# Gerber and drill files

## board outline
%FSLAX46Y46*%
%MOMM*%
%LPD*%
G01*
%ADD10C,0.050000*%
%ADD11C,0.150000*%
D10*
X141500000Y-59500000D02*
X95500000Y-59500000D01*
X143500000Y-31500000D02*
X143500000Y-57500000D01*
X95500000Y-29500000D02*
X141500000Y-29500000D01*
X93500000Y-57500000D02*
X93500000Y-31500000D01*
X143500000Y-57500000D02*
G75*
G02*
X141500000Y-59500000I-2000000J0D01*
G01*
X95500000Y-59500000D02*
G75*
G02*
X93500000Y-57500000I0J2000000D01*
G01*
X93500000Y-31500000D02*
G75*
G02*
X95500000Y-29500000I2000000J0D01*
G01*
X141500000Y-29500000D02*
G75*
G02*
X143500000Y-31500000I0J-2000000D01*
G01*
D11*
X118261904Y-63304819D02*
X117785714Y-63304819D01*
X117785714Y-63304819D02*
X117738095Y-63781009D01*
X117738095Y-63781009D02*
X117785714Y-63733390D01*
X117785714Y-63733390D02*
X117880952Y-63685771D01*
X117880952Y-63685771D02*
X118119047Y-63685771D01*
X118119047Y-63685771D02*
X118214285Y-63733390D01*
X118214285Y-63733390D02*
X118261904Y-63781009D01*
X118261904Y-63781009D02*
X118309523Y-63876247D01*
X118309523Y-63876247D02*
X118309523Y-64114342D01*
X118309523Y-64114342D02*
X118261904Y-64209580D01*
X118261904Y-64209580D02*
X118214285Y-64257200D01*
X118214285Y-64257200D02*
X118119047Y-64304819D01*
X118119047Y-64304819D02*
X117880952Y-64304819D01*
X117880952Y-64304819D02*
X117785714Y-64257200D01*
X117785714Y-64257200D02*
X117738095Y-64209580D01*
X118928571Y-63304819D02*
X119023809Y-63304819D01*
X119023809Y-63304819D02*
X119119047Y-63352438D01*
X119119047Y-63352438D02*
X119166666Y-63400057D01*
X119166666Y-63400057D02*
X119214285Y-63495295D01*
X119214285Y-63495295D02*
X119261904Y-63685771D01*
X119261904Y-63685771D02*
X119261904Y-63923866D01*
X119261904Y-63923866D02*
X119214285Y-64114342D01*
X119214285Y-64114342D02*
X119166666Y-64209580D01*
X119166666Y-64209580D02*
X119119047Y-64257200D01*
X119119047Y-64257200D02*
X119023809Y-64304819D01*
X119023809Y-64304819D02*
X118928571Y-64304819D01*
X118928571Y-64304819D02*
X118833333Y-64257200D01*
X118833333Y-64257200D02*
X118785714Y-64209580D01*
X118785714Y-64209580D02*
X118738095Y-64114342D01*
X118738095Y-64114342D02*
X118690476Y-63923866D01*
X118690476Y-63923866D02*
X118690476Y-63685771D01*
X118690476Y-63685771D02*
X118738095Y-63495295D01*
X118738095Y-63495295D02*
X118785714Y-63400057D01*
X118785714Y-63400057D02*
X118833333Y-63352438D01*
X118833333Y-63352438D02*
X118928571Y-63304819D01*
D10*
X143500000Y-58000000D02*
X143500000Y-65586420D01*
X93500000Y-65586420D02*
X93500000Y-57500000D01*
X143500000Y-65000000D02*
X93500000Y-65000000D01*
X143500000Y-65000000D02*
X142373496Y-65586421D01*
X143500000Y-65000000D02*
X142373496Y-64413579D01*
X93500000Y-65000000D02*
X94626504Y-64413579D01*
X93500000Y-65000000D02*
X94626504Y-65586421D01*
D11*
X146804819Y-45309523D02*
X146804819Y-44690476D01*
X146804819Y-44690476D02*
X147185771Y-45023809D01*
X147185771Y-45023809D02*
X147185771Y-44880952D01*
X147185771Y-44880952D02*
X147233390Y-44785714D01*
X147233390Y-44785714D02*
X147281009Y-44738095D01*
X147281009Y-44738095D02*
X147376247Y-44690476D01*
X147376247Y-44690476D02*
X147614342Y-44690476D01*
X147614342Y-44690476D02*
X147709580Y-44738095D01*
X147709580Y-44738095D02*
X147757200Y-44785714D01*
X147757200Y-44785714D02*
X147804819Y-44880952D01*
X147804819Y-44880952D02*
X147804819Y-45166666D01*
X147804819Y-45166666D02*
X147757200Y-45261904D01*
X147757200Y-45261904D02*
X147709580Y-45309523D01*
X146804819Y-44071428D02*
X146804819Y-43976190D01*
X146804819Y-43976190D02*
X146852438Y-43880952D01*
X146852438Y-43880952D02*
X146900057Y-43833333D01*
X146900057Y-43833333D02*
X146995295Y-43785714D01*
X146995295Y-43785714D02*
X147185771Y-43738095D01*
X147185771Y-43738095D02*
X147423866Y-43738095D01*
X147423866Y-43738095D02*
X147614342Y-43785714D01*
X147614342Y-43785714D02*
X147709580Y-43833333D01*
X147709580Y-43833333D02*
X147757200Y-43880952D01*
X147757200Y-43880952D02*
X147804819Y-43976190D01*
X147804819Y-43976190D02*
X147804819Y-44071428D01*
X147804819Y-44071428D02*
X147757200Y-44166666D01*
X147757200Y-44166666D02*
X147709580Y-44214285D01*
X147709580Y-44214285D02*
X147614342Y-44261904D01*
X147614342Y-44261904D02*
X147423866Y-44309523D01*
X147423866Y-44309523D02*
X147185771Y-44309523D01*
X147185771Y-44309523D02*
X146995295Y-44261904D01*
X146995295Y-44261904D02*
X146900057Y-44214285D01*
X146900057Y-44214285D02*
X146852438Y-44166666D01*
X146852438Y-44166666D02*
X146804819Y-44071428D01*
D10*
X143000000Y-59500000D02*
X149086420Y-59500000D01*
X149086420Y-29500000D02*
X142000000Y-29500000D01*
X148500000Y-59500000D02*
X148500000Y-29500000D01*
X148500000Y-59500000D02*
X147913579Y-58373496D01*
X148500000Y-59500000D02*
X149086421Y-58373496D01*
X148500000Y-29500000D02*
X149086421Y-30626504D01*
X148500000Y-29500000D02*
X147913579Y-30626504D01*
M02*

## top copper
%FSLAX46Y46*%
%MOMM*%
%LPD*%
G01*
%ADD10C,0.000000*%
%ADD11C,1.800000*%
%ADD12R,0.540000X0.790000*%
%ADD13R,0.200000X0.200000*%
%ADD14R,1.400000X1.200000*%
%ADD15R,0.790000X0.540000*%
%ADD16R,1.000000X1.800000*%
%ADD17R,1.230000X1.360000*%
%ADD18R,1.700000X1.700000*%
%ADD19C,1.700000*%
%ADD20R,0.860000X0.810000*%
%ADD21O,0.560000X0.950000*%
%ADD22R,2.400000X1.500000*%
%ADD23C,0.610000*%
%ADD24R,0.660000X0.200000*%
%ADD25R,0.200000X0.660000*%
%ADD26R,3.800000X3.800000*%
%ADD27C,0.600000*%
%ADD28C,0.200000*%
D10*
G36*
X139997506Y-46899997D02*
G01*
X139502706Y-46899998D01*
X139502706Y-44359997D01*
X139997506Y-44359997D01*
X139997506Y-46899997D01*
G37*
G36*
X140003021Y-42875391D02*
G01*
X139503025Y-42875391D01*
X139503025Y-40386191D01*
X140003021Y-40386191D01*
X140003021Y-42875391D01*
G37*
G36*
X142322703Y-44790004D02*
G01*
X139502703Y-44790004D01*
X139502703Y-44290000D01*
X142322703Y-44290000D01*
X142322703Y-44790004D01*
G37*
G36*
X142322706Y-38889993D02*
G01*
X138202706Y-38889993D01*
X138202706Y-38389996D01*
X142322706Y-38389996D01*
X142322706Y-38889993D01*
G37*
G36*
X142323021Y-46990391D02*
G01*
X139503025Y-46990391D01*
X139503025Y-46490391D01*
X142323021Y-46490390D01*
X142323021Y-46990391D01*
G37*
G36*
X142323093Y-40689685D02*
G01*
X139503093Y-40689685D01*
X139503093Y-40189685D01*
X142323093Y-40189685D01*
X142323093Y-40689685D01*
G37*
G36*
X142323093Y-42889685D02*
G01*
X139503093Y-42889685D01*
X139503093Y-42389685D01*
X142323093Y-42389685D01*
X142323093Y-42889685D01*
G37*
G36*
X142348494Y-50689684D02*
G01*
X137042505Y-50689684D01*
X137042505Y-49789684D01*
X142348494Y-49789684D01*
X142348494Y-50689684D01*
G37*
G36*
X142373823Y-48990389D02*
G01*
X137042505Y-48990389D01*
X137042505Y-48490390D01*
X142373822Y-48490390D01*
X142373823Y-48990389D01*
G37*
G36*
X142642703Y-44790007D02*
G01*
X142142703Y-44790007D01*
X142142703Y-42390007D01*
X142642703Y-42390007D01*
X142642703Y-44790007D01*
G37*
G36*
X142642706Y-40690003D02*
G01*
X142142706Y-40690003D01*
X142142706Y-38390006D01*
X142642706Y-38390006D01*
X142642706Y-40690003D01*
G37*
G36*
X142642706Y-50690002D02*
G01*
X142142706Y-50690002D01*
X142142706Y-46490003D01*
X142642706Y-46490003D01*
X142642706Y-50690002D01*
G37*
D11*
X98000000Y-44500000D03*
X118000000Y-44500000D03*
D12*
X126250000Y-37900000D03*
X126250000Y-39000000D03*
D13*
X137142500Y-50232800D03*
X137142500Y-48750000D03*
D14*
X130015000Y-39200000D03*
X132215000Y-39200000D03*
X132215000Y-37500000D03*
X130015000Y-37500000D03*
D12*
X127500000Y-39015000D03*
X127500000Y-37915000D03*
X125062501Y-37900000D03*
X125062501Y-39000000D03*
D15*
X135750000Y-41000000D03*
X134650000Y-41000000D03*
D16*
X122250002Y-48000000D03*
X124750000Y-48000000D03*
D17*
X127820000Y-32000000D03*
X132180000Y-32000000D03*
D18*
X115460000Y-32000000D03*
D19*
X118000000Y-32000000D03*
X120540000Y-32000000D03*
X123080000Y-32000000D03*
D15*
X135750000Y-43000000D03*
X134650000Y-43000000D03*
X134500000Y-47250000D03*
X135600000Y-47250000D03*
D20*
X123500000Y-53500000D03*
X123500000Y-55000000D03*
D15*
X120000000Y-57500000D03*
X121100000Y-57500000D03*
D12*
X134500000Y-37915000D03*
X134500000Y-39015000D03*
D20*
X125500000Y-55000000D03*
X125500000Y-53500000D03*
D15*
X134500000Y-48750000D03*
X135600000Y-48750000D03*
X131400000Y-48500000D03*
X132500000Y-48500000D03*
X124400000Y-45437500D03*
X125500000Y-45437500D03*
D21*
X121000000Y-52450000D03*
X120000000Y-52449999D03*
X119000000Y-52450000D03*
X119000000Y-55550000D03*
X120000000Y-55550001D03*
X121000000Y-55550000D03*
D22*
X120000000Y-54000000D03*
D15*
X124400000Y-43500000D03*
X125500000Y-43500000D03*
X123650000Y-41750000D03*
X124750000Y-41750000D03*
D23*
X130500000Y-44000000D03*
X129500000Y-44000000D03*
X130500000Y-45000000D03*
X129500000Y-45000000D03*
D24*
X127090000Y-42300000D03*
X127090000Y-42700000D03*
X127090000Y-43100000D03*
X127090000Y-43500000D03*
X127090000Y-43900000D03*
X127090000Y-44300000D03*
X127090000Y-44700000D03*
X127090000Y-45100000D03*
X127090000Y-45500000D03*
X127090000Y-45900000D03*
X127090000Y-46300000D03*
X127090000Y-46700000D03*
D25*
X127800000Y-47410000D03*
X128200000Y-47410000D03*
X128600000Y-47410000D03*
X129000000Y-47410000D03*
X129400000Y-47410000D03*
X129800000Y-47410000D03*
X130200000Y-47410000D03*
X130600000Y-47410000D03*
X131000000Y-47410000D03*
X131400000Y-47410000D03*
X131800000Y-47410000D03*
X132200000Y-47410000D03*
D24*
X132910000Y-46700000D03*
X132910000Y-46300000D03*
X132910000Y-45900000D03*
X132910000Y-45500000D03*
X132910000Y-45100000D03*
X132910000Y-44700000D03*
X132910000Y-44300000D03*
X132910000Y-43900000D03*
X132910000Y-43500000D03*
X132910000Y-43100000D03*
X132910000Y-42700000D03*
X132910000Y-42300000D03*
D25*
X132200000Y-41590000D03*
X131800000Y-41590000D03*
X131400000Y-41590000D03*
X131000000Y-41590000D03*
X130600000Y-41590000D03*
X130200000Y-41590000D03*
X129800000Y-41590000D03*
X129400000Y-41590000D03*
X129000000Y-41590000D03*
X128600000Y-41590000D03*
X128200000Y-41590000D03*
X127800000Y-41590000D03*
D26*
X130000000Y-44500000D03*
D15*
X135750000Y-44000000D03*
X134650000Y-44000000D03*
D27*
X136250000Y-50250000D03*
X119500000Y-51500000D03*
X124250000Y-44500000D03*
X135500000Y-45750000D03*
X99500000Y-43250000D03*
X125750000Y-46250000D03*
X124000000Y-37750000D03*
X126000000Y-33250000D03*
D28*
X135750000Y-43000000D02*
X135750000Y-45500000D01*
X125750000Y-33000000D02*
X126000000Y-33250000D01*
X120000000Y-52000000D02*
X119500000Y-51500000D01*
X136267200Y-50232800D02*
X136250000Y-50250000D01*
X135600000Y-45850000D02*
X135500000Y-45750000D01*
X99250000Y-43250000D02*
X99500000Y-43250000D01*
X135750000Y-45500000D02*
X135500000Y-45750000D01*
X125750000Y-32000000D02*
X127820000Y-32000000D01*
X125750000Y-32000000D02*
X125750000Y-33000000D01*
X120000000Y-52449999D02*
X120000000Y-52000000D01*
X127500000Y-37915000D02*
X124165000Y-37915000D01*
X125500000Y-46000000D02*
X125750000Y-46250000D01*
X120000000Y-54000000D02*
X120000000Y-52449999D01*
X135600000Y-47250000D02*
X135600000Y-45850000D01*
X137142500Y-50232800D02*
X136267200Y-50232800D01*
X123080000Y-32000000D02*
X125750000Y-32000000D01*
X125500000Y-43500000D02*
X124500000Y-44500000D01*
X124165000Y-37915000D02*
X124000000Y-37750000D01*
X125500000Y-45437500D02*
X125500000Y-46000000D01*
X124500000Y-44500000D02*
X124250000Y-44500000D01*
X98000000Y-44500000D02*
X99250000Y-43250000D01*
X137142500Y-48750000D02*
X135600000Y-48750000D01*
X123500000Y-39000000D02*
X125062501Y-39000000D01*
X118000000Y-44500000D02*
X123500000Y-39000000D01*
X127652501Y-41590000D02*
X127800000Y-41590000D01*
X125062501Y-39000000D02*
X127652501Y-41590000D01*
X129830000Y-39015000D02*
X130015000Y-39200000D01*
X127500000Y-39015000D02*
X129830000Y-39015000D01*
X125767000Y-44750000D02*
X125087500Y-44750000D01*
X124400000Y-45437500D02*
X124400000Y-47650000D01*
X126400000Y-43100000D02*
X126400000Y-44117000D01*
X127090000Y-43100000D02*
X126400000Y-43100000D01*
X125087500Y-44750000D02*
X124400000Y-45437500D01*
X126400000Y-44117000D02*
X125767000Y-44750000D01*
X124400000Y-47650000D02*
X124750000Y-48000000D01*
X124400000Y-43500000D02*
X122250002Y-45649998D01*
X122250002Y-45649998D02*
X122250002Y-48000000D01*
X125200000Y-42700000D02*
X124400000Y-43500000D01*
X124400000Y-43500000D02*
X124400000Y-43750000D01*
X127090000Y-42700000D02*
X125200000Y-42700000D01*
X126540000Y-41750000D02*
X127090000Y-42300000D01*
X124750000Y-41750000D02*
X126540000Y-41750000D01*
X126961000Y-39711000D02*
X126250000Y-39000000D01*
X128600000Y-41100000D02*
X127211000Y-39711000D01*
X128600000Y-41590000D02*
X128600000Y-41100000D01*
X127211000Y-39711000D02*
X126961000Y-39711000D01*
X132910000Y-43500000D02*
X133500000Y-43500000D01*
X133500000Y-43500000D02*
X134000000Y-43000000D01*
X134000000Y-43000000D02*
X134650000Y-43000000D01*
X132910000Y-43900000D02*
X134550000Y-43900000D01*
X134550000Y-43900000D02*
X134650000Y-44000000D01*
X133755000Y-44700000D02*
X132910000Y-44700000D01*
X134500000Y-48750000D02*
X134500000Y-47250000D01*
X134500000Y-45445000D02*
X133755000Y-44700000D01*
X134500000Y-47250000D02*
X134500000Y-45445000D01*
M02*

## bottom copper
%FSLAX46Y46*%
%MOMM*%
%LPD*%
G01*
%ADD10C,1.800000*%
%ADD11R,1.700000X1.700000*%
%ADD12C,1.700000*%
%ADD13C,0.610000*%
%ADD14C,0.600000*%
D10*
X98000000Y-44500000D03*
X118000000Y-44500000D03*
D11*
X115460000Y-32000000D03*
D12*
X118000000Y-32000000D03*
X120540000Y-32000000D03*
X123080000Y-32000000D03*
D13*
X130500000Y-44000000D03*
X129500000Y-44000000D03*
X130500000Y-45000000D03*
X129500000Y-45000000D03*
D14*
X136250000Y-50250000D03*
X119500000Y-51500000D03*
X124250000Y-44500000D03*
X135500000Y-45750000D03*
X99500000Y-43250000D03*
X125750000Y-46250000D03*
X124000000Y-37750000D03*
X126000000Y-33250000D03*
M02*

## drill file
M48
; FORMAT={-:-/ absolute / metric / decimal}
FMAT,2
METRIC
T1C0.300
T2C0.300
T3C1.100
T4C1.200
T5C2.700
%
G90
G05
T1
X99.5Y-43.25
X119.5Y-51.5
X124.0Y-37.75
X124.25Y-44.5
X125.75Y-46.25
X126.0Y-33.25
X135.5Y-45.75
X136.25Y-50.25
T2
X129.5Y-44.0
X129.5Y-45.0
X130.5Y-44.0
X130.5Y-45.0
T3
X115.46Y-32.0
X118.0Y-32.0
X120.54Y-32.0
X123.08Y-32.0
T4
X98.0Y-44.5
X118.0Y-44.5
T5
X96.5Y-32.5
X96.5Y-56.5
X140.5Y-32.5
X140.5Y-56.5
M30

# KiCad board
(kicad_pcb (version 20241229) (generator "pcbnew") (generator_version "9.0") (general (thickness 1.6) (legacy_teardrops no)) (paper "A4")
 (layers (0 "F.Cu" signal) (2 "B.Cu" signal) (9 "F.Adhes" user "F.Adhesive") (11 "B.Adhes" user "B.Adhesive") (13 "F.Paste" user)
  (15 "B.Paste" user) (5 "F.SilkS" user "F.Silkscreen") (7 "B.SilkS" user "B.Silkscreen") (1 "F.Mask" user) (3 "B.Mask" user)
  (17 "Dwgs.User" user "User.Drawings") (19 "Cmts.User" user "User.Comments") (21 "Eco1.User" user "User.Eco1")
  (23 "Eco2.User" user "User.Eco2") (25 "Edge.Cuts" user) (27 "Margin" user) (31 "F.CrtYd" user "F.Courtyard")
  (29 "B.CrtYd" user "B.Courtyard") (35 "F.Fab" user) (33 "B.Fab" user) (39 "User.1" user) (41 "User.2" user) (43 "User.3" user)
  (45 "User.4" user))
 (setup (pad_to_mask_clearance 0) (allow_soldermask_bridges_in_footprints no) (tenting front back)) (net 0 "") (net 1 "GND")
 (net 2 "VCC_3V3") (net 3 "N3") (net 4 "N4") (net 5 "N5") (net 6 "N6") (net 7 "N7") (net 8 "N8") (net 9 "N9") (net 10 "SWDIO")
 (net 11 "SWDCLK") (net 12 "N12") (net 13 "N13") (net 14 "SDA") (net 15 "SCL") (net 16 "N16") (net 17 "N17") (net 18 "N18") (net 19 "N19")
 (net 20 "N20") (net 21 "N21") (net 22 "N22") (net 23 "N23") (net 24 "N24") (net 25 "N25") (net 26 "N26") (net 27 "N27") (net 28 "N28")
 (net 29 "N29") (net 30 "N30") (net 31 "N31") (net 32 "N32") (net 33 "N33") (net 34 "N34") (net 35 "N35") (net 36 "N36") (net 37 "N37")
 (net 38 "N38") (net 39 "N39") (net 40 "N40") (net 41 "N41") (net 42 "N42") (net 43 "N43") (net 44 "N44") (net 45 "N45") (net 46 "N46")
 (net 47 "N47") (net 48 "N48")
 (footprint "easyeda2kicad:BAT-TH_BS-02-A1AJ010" (layer "F.Cu") (at 108 44.5)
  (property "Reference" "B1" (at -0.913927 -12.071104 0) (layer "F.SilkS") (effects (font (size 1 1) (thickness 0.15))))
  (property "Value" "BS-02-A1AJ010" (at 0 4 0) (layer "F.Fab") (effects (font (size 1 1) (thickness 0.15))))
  (pad "1" thru_hole circle (at -10 0) (size 1.8 1.8) (drill 1.199998) (layers "*.Cu" "*.Mask") (remove_unused_layers no) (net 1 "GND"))
  (pad "2" thru_hole circle (at 10 0) (size 1.8 1.8) (drill 1.199998) (layers "*.Cu" "*.Mask") (remove_unused_layers no) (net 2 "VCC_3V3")))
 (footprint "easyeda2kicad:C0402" (layer "F.Cu") (at 126.25 38.45 -90)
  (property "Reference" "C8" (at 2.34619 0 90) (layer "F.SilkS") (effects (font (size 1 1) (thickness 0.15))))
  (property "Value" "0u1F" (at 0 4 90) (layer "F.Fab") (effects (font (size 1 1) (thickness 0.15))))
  (pad "1" smd rect (at -0.55 0 270) (size 0.79 0.54) (layers "F.Cu" "F.Mask" "F.Paste") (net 1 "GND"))
  (pad "2" smd rect (at 0.55 0 270) (size 0.79 0.54) (layers "F.Cu" "F.Mask" "F.Paste") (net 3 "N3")))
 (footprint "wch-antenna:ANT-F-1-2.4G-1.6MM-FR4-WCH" (layer "F.Cu") (at 140 44.6225 -90)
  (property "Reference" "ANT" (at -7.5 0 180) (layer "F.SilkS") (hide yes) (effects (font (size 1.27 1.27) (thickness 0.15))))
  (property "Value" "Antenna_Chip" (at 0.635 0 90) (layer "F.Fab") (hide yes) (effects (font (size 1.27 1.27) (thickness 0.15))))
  (fp_poly
   (pts (xy 2.277497 0.002494) (xy -0.262503 0.002494) (xy -0.262503 0.497294) (xy 2.277498 0.497294)) (stroke (width 0) (type solid))
   (fill yes) (layer "F.Cu"))
  (fp_poly
   (pts (xy -1.747109 -0.003021) (xy -4.236309 -0.003021) (xy -4.236309 0.496975) (xy -1.747109 0.496975)) (stroke (width 0) (type solid))
   (fill yes) (layer "F.Cu"))
  (fp_poly
   (pts (xy 0.167504 -2.322703) (xy -0.3325 -2.322703) (xy -0.3325 0.497297) (xy 0.167504 0.497297)) (stroke (width 0) (type solid))
   (fill yes) (layer "F.Cu"))
  (fp_poly
   (pts (xy -5.732507 -2.322706) (xy -6.232504 -2.322706) (xy -6.232504 1.797294) (xy -5.732507 1.797294)) (stroke (width 0) (type solid))
   (fill yes) (layer "F.Cu"))
  (fp_poly
   (pts (xy 2.367891 -2.323021) (xy 1.86789 -2.323021) (xy 1.867891 0.496975) (xy 2.367891 0.496975)) (stroke (width 0) (type solid))
   (fill yes) (layer "F.Cu"))
  (fp_poly
   (pts (xy -3.932815 -2.323093) (xy -4.432815 -2.323093) (xy -4.432815 0.496907) (xy -3.932815 0.496907)) (stroke (width 0) (type solid))
   (fill yes) (layer "F.Cu"))
  (fp_poly
   (pts (xy -1.732815 -2.323093) (xy -2.232815 -2.323093) (xy -2.232815 0.496907) (xy -1.732815 0.496907)) (stroke (width 0) (type solid))
   (fill yes) (layer "F.Cu"))
  (fp_poly
   (pts (xy 6.067184 -2.348494) (xy 5.167184 -2.348494) (xy 5.167184 2.957495) (xy 6.067184 2.957495)) (stroke (width 0) (type solid))
   (fill yes) (layer "F.Cu"))
  (fp_poly
   (pts (xy 4.367889 -2.373823) (xy 3.86789 -2.373822) (xy 3.86789 2.957495) (xy 4.367889 2.957495)) (stroke (width 0) (type solid))
   (fill yes) (layer "F.Cu"))
  (fp_poly
   (pts (xy 0.167507 -2.642703) (xy -2.232493 -2.642703) (xy -2.232493 -2.142703) (xy 0.167507 -2.142703)) (stroke (width 0) (type solid))
   (fill yes) (layer "F.Cu"))
  (fp_poly
   (pts (xy -3.932497 -2.642706) (xy -6.232494 -2.642706) (xy -6.232494 -2.142706) (xy -3.932497 -2.142706)) (stroke (width 0) (type solid))
   (fill yes) (layer "F.Cu"))
  (fp_poly
   (pts (xy 6.067502 -2.642706) (xy 1.867503 -2.642706) (xy 1.867503 -2.142706) (xy 6.067502 -2.142706)) (stroke (width 0) (type solid))
   (fill yes) (layer "F.Cu"))
  (pad "1" smd rect (at 5.6103 2.8575) (size 0.2 0.2) (layers "F.Cu") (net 1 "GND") (solder_mask_margin 0.1016))
  (pad "2" smd rect (at 4.1275 2.8575) (size 0.2 0.2) (layers "F.Cu") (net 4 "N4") (solder_mask_margin 0.1016)))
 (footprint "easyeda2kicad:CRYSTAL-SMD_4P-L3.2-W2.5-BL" (layer "F.Cu") (at 131.115 38.35)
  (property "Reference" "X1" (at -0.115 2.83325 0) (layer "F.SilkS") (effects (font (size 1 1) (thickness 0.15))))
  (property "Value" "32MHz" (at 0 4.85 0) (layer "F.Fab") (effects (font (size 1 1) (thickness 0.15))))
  (pad "1" smd rect (at -1.1 0.85) (size 1.4 1.2) (layers "F.Cu" "F.Mask" "F.Paste") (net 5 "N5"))
  (pad "2" smd rect (at 1.1 0.85) (size 1.4 1.2) (layers "F.Cu" "F.Mask" "F.Paste") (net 1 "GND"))
  (pad "3" smd rect (at 1.1 -0.85) (size 1.4 1.2) (layers "F.Cu" "F.Mask" "F.Paste") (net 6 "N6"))
  (pad "4" smd rect (at -1.1 -0.85) (size 1.4 1.2) (layers "F.Cu" "F.Mask" "F.Paste") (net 1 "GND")))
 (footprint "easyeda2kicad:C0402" (layer "F.Cu") (at 127.5 38.465 90)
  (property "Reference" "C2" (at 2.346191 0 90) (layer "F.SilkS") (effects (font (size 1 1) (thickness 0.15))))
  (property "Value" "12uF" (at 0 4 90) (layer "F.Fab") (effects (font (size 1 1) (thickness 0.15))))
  (pad "1" smd rect (at -0.55 0 90) (size 0.79 0.54) (layers "F.Cu" "F.Mask" "F.Paste") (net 5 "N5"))
  (pad "2" smd rect (at 0.55 0 90) (size 0.79 0.54) (layers "F.Cu" "F.Mask" "F.Paste") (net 1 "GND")))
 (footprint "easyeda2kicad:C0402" (layer "F.Cu") (at 125.062501 38.45 -90)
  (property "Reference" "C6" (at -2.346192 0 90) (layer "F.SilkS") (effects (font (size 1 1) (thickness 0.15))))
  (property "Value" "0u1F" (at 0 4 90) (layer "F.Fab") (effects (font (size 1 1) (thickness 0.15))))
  (pad "1" smd rect (at -0.55 0 270) (size 0.79 0.54) (layers "F.Cu" "F.Mask" "F.Paste") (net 1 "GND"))
  (pad "2" smd rect (at 0.55 0 270) (size 0.79 0.54) (layers "F.Cu" "F.Mask" "F.Paste") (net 2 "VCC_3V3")))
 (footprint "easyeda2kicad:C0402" (layer "F.Cu") (at 135.2 41 180)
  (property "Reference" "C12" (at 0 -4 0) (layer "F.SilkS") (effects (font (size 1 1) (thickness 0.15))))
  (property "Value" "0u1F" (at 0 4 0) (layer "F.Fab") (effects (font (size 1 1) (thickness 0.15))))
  (pad "1" smd rect (at -0.55 0 180) (size 0.79 0.54) (layers "F.Cu" "F.Mask" "F.Paste") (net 1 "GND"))
  (pad "2" smd rect (at 0.55 0 180) (size 0.79 0.54) (layers "F.Cu" "F.Mask" "F.Paste") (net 2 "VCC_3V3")))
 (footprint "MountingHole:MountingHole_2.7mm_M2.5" (layer "F.Cu") (at 140.5 32.5)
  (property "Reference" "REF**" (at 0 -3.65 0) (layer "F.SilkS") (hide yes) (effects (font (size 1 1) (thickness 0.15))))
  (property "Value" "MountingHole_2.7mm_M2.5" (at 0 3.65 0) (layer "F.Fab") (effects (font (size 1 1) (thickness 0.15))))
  (pad "" np_thru_hole circle (at 0 0) (size 2.7 2.7) (drill 2.7) (layers "*.Cu" "*.Mask")))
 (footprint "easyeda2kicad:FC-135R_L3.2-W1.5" (layer "F.Cu") (at 123.500001 48)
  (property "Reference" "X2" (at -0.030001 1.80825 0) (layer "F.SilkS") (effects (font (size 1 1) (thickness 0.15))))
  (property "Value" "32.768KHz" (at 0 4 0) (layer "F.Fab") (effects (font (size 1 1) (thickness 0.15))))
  (pad "1" smd rect (at -1.249999 0 90) (size 1.8 1) (layers "F.Cu" "F.Mask" "F.Paste") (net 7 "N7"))
  (pad "2" smd rect (at 1.249999 0 90) (size 1.8 1) (layers "F.Cu" "F.Mask" "F.Paste") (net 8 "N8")))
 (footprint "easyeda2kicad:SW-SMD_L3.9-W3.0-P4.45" (layer "F.Cu") (at 130 32)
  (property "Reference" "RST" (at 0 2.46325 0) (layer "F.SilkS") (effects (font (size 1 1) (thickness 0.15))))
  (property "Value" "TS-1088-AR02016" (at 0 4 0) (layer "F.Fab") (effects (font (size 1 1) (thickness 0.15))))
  (pad "1" smd rect (at -2.18 0) (size 1.23 1.36) (layers "F.Cu" "F.Mask" "F.Paste") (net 1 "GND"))
  (pad "2" smd rect (at 2.18 0) (size 1.23 1.36) (layers "F.Cu" "F.Mask" "F.Paste") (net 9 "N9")))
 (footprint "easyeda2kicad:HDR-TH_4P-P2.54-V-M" (layer "F.Cu") (at 119.27 32)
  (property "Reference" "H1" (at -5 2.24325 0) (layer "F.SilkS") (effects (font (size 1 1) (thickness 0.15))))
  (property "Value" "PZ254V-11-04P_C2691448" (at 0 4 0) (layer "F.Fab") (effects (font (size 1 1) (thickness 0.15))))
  (pad "1" thru_hole rect (at -3.81 0) (size 1.7 1.7) (drill 1.100023) (layers "*.Cu" "*.Mask") (remove_unused_layers no) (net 2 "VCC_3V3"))
  (pad "2" thru_hole circle (at -1.27 0) (size 1.7 1.7) (drill 1.100023) (layers "*.Cu" "*.Mask") (remove_unused_layers no) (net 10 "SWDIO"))
  (pad "3" thru_hole circle (at 1.27 0) (size 1.7 1.7) (drill 1.100023) (layers "*.Cu" "*.Mask") (remove_unused_layers no) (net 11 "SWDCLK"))
  (pad "4" thru_hole circle (at 3.81 0) (size 1.7 1.7) (drill 1.100023) (layers "*.Cu" "*.Mask") (remove_unused_layers no) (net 1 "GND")))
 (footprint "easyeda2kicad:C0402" (layer "F.Cu") (at 135.2 43 180)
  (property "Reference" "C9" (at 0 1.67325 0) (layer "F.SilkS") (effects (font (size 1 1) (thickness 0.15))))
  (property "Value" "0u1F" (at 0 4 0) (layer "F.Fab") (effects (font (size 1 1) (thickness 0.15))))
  (pad "1" smd rect (at -0.55 0 180) (size 0.79 0.54) (layers "F.Cu" "F.Mask" "F.Paste") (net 1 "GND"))
  (pad "2" smd rect (at 0.55 0 180) (size 0.79 0.54) (layers "F.Cu" "F.Mask" "F.Paste") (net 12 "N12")))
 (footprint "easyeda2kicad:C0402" (layer "F.Cu") (at 135.05 47.25)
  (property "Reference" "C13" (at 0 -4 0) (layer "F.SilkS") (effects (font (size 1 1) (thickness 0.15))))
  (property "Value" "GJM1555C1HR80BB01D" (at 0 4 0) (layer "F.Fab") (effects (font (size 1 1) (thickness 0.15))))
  (pad "1" smd rect (at -0.55 0) (size 0.79 0.54) (layers "F.Cu" "F.Mask" "F.Paste") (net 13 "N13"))
  (pad "2" smd rect (at 0.55 0) (size 0.79 0.54) (layers "F.Cu" "F.Mask" "F.Paste") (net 1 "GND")))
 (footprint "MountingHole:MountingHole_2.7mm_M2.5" (layer "F.Cu") (at 140.5 56.5)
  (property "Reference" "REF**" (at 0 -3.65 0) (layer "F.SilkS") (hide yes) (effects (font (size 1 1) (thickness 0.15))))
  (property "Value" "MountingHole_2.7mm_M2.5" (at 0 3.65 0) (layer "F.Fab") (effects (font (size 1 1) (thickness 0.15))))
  (pad "" np_thru_hole circle (at 0 0) (size 2.7 2.7) (drill 2.7) (layers "*.Cu" "*.Mask")))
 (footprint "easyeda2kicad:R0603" (layer "F.Cu") (at 123.5 54.25 -90)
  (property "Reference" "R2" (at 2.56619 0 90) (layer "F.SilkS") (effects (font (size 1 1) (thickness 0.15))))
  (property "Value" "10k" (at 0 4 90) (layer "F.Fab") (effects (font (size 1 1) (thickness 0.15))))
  (pad "1" smd rect (at -0.75 0 270) (size 0.81 0.86) (layers "F.Cu" "F.Mask" "F.Paste") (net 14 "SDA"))
  (pad "2" smd rect (at 0.75 0 270) (size 0.81 0.86) (layers "F.Cu" "F.Mask" "F.Paste") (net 2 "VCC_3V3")))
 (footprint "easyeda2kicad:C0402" (layer "F.Cu") (at 120.55 57.5)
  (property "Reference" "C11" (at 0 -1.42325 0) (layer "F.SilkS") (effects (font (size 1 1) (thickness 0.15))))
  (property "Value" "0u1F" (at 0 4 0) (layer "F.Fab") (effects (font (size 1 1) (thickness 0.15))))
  (pad "1" smd rect (at -0.55 0) (size 0.79 0.54) (layers "F.Cu" "F.Mask" "F.Paste") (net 1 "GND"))
  (pad "2" smd rect (at 0.55 0) (size 0.79 0.54) (layers "F.Cu" "F.Mask" "F.Paste") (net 2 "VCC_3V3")))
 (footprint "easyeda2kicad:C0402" (layer "F.Cu") (at 134.5 38.465 -90)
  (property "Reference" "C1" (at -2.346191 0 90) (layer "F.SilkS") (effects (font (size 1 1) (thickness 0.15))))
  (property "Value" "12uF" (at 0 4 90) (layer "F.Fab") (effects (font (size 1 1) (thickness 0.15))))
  (pad "1" smd rect (at -0.55 0 270) (size 0.79 0.54) (layers "F.Cu" "F.Mask" "F.Paste") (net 6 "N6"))
  (pad "2" smd rect (at 0.55 0 270) (size 0.79 0.54) (layers "F.Cu" "F.Mask" "F.Paste") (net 1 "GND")))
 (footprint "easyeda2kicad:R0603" (layer "F.Cu") (at 125.5 54.25 90)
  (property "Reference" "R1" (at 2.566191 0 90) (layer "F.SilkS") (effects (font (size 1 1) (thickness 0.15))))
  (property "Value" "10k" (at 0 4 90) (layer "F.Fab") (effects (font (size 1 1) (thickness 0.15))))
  (pad "1" smd rect (at -0.75 0 90) (size 0.81 0.86) (layers "F.Cu" "F.Mask" "F.Paste") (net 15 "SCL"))
  (pad "2" smd rect (at 0.75 0 90) (size 0.81 0.86) (layers "F.Cu" "F.Mask" "F.Paste") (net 2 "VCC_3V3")))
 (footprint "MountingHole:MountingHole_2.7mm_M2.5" (layer "F.Cu") (at 96.5 32.5)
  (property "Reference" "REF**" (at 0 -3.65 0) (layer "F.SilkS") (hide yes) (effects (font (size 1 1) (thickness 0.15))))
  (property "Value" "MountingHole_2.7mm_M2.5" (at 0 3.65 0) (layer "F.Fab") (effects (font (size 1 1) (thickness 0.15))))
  (pad "" np_thru_hole circle (at 0 0) (size 2.7 2.7) (drill 2.7) (layers "*.Cu" "*.Mask")))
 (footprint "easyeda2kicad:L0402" (layer "F.Cu") (at 135.05 48.75)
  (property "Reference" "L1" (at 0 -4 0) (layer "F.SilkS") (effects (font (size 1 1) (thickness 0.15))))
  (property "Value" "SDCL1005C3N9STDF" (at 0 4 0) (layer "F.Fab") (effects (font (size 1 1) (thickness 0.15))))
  (pad "1" smd rect (at -0.55 0) (size 0.79 0.54) (layers "F.Cu" "F.Mask" "F.Paste") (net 13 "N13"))
  (pad "2" smd rect (at 0.55 0) (size 0.79 0.54) (layers "F.Cu" "F.Mask" "F.Paste") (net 4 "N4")))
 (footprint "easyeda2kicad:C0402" (layer "F.Cu") (at 131.95 48.5)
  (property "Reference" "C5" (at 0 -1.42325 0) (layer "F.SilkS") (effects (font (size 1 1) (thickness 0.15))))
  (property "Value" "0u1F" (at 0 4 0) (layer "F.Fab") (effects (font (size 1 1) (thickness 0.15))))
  (pad "1" smd rect (at -0.55 0) (size 0.79 0.54) (layers "F.Cu" "F.Mask" "F.Paste") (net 1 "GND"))
  (pad "2" smd rect (at 0.55 0) (size 0.79 0.54) (layers "F.Cu" "F.Mask" "F.Paste") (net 2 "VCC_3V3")))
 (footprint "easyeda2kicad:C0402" (layer "F.Cu") (at 124.95 45.4375)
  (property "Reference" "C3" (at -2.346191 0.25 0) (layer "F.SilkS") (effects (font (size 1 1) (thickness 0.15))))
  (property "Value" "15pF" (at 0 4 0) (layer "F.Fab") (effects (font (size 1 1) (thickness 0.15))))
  (pad "1" smd rect (at -0.55 0) (size 0.79 0.54) (layers "F.Cu" "F.Mask" "F.Paste") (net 8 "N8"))
  (pad "2" smd rect (at 0.55 0) (size 0.79 0.54) (layers "F.Cu" "F.Mask" "F.Paste") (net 1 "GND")))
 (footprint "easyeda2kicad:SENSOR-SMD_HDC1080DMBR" (layer "F.Cu") (at 120 54 -90)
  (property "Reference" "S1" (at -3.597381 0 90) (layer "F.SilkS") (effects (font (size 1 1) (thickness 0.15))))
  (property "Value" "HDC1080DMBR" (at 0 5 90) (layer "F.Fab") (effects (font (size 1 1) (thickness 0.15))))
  (pad "1" smd oval (at -1.55 -1 270) (size 0.95 0.56) (layers "F.Cu" "F.Mask" "F.Paste") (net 14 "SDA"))
  (pad "2" smd oval (at -1.550001 0 270) (size 0.95 0.56) (layers "F.Cu" "F.Mask" "F.Paste") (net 1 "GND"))
  (pad "3" smd oval (at -1.55 1 270) (size 0.95 0.56) (layers "F.Cu" "F.Mask" "F.Paste") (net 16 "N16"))
  (pad "4" smd oval (at 1.55 1 270) (size 0.95 0.56) (layers "F.Cu" "F.Mask" "F.Paste") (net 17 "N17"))
  (pad "5" smd oval (at 1.550001 0 270) (size 0.95 0.56) (layers "F.Cu" "F.Mask" "F.Paste") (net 2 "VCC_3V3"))
  (pad "6" smd oval (at 1.55 -1 270) (size 0.95 0.56) (layers "F.Cu" "F.Mask" "F.Paste") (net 15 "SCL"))
  (pad "7" smd rect (at 0 0 270) (size 1.5 2.4) (layers "F.Cu" "F.Mask" "F.Paste") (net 1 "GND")))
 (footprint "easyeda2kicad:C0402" (layer "F.Cu") (at 124.95 43.5)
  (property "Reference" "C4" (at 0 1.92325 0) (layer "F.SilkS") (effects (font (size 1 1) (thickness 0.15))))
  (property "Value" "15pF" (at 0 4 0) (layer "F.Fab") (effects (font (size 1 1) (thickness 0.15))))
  (pad "1" smd rect (at -0.55 0) (size 0.79 0.54) (layers "F.Cu" "F.Mask" "F.Paste") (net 7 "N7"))
  (pad "2" smd rect (at 0.55 0) (size 0.79 0.54) (layers "F.Cu" "F.Mask" "F.Paste") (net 1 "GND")))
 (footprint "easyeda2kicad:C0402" (layer "F.Cu") (at 124.2 41.75)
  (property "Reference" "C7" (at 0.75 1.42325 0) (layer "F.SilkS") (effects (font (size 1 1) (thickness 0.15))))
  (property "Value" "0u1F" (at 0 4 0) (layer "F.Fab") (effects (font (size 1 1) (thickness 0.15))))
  (pad "1" smd rect (at -0.55 0) (size 0.79 0.54) (layers "F.Cu" "F.Mask" "F.Paste") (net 1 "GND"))
  (pad "2" smd rect (at 0.55 0) (size 0.79 0.54) (layers "F.Cu" "F.Mask" "F.Paste") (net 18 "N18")))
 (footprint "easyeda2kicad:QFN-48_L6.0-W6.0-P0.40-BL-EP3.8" (layer "F.Cu") (at 130 44.5 -90)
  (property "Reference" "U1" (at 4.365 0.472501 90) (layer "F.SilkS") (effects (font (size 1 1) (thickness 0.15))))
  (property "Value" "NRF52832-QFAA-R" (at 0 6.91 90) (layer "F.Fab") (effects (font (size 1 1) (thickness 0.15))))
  (pad "" thru_hole circle (at -0.5 -0.5 270) (size 0.61 0.61) (drill 0.3) (layers "*.Cu" "*.Paste" "*.Mask") (remove_unused_layers no))
  (pad "" thru_hole circle (at -0.5 0.5 270) (size 0.61 0.61) (drill 0.3) (layers "*.Cu" "*.Paste" "*.Mask") (remove_unused_layers no))
  (pad "" thru_hole circle (at 0.5 -0.5 270) (size 0.61 0.61) (drill 0.3) (layers "*.Cu" "*.Paste" "*.Mask") (remove_unused_layers no))
  (pad "" thru_hole circle (at 0.5 0.5 270) (size 0.61 0.61) (drill 0.3) (layers "*.Cu" "*.Paste" "*.Mask") (remove_unused_layers no))
  (pad "1" smd rect (at -2.2 2.91 270) (size 0.2 0.66) (layers "F.Cu" "F.Mask" "F.Paste") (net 18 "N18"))
  (pad "2" smd rect (at -1.8 2.91 270) (size 0.2 0.66) (layers "F.Cu" "F.Mask" "F.Paste") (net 7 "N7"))
  (pad "3" smd rect (at -1.4 2.91 270) (size 0.2 0.66) (layers "F.Cu" "F.Mask" "F.Paste") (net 8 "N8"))
  (pad "4" smd rect (at -1 2.91 270) (size 0.2 0.66) (layers "F.Cu" "F.Mask" "F.Paste") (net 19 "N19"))
  (pad "5" smd rect (at -0.6 2.91 270) (size 0.2 0.66) (layers "F.Cu" "F.Mask" "F.Paste") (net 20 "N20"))
  (pad "6" smd rect (at -0.2 2.91 270) (size 0.2 0.66) (layers "F.Cu" "F.Mask" "F.Paste") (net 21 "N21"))
  (pad "7" smd rect (at 0.2 2.91 270) (size 0.2 0.66) (layers "F.Cu" "F.Mask" "F.Paste") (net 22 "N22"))
  (pad "8" smd rect (at 0.6 2.91 270) (size 0.2 0.66) (layers "F.Cu" "F.Mask" "F.Paste") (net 14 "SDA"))
  (pad "9" smd rect (at 1 2.91 270) (size 0.2 0.66) (layers "F.Cu" "F.Mask" "F.Paste") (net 15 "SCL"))
  (pad "10" smd rect (at 1.4 2.91 270) (size 0.2 0.66) (layers "F.Cu" "F.Mask" "F.Paste") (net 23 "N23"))
  (pad "11" smd rect (at 1.8 2.91 270) (size 0.2 0.66) (layers "F.Cu" "F.Mask" "F.Paste") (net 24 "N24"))
  (pad "12" smd rect (at 2.2 2.91 270) (size 0.2 0.66) (layers "F.Cu" "F.Mask" "F.Paste") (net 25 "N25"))
  (pad "13" smd rect (at 2.91 2.2 270) (size 0.66 0.2) (layers "F.Cu" "F.Mask" "F.Paste") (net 2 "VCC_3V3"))
  (pad "14" smd rect (at 2.91 1.8 270) (size 0.66 0.2) (layers "F.Cu" "F.Mask" "F.Paste") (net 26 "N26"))
  (pad "15" smd rect (at 2.91 1.4 270) (size 0.66 0.2) (layers "F.Cu" "F.Mask" "F.Paste") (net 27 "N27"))
  (pad "16" smd rect (at 2.91 1 270) (size 0.66 0.2) (layers "F.Cu" "F.Mask" "F.Paste") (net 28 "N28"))
  (pad "17" smd rect (at 2.91 0.6 270) (size 0.66 0.2) (layers "F.Cu" "F.Mask" "F.Paste") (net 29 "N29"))
  (pad "18" smd rect (at 2.91 0.2 270) (size 0.66 0.2) (layers "F.Cu" "F.Mask" "F.Paste") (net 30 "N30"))
  (pad "19" smd rect (at 2.91 -0.2 270) (size 0.66 0.2) (layers "F.Cu" "F.Mask" "F.Paste") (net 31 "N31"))
  (pad "20" smd rect (at 2.91 -0.6 270) (size 0.66 0.2) (layers "F.Cu" "F.Mask" "F.Paste") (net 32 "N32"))
  (pad "21" smd rect (at 2.91 -1 270) (size 0.66 0.2) (layers "F.Cu" "F.Mask" "F.Paste") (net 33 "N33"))
  (pad "22" smd rect (at 2.91 -1.4 270) (size 0.66 0.2) (layers "F.Cu" "F.Mask" "F.Paste") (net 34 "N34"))
  (pad "23" smd rect (at 2.91 -1.8 270) (size 0.66 0.2) (layers "F.Cu" "F.Mask" "F.Paste") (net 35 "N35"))
  (pad "24" smd rect (at 2.91 -2.2 270) (size 0.66 0.2) (layers "F.Cu" "F.Mask" "F.Paste") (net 9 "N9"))
  (pad "25" smd rect (at 2.2 -2.91 270) (size 0.2 0.66) (layers "F.Cu" "F.Mask" "F.Paste") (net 11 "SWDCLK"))
  (pad "26" smd rect (at 1.8 -2.91 270) (size 0.2 0.66) (layers "F.Cu" "F.Mask" "F.Paste") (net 10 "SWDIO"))
  (pad "27" smd rect (at 1.4 -2.91 270) (size 0.2 0.66) (layers "F.Cu" "F.Mask" "F.Paste") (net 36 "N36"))
  (pad "28" smd rect (at 1 -2.91 270) (size 0.2 0.66) (layers "F.Cu" "F.Mask" "F.Paste") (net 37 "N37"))
  (pad "29" smd rect (at 0.6 -2.91 270) (size 0.2 0.66) (layers "F.Cu" "F.Mask" "F.Paste") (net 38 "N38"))
  (pad "30" smd rect (at 0.2 -2.91 270) (size 0.2 0.66) (layers "F.Cu" "F.Mask" "F.Paste") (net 13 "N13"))
  (pad "31" smd rect (at -0.2 -2.91 270) (size 0.2 0.66) (layers "F.Cu" "F.Mask" "F.Paste") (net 1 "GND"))
  (pad "32" smd rect (at -0.6 -2.91 270) (size 0.2 0.66) (layers "F.Cu" "F.Mask" "F.Paste") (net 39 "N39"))
  (pad "33" smd rect (at -1 -2.91 270) (size 0.2 0.66) (layers "F.Cu" "F.Mask" "F.Paste") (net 12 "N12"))
  (pad "34" smd rect (at -1.4 -2.91 270) (size 0.2 0.66) (layers "F.Cu" "F.Mask" "F.Paste") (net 5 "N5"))
  (pad "35" smd rect (at -1.8 -2.91 270) (size 0.2 0.66) (layers "F.Cu" "F.Mask" "F.Paste") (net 6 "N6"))
  (pad "36" smd rect (at -2.2 -2.91 270) (size 0.2 0.66) (layers "F.Cu" "F.Mask" "F.Paste") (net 2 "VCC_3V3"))
  (pad "37" smd rect (at -2.91 -2.2 270) (size 0.66 0.2) (layers "F.Cu" "F.Mask" "F.Paste") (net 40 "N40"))
  (pad "38" smd rect (at -2.91 -1.8 270) (size 0.66 0.2) (layers "F.Cu" "F.Mask" "F.Paste") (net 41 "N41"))
  (pad "39" smd rect (at -2.91 -1.4 270) (size 0.66 0.2) (layers "F.Cu" "F.Mask" "F.Paste") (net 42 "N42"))
  (pad "40" smd rect (at -2.91 -1 270) (size 0.66 0.2) (layers "F.Cu" "F.Mask" "F.Paste") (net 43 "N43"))
  (pad "41" smd rect (at -2.91 -0.6 270) (size 0.66 0.2) (layers "F.Cu" "F.Mask" "F.Paste") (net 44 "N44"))
  (pad "42" smd rect (at -2.91 -0.2 270) (size 0.66 0.2) (layers "F.Cu" "F.Mask" "F.Paste") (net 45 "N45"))
  (pad "43" smd rect (at -2.91 0.2 270) (size 0.66 0.2) (layers "F.Cu" "F.Mask" "F.Paste") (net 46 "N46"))
  (pad "44" smd rect (at -2.91 0.6 270) (size 0.66 0.2) (layers "F.Cu" "F.Mask" "F.Paste") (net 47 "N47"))
  (pad "45" smd rect (at -2.91 1 270) (size 0.66 0.2) (layers "F.Cu" "F.Mask" "F.Paste") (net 1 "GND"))
  (pad "46" smd rect (at -2.91 1.4 270) (size 0.66 0.2) (layers "F.Cu" "F.Mask" "F.Paste") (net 3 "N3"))
  (pad "47" smd rect (at -2.91 1.8 270) (size 0.66 0.2) (layers "F.Cu" "F.Mask" "F.Paste") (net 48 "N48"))
  (pad "48" smd rect (at -2.91 2.2 270) (size 0.66 0.2) (layers "F.Cu" "F.Mask" "F.Paste") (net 2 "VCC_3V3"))
  (pad "49" smd rect (at 0 0 270) (size 3.8 3.8) (layers "F.Cu" "F.Mask" "F.Paste") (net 1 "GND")))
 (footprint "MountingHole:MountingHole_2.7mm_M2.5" (layer "F.Cu") (at 96.5 56.5)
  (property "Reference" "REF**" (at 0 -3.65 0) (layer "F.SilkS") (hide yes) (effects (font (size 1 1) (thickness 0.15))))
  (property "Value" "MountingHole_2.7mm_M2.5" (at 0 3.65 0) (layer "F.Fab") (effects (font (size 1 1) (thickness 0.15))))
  (pad "" np_thru_hole circle (at 0 0) (size 2.7 2.7) (drill 2.7) (layers "*.Cu" "*.Mask")))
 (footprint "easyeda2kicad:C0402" (layer "F.Cu") (at 135.2 44 180)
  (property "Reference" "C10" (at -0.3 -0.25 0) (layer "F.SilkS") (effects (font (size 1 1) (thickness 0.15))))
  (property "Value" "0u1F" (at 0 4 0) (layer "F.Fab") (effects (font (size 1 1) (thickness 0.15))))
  (pad "1" smd rect (at -0.55 0 180) (size 0.79 0.54) (layers "F.Cu" "F.Mask" "F.Paste") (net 1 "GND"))
  (pad "2" smd rect (at 0.55 0 180) (size 0.79 0.54) (layers "F.Cu" "F.Mask" "F.Paste") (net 39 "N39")))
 (gr_line (start 141.5 59.5) (end 95.5 59.5) (stroke (width 0.05) (type default)) (layer "Edge.Cuts"))
 (gr_line (start 143.5 31.5) (end 143.5 57.5) (stroke (width 0.05) (type default)) (layer "Edge.Cuts"))
 (gr_line (start 95.5 29.5) (end 141.5 29.5) (stroke (width 0.05) (type default)) (layer "Edge.Cuts"))
 (gr_line (start 93.5 57.5) (end 93.5 31.5) (stroke (width 0.05) (type default)) (layer "Edge.Cuts"))
 (gr_arc (start 143.5 57.5) (mid 142.914214 58.914214) (end 141.5 59.5) (stroke (width 0.05) (type default)) (layer "Edge.Cuts"))
 (gr_arc (start 95.5 59.5) (mid 94.085786 58.914214) (end 93.5 57.5) (stroke (width 0.05) (type default)) (layer "Edge.Cuts"))
 (gr_arc (start 93.5 31.5) (mid 94.085786 30.085786) (end 95.5 29.5) (stroke (width 0.05) (type default)) (layer "Edge.Cuts"))
 (gr_arc (start 141.5 29.5) (mid 142.914214 30.085786) (end 143.5 31.5) (stroke (width 0.05) (type default)) (layer "Edge.Cuts"))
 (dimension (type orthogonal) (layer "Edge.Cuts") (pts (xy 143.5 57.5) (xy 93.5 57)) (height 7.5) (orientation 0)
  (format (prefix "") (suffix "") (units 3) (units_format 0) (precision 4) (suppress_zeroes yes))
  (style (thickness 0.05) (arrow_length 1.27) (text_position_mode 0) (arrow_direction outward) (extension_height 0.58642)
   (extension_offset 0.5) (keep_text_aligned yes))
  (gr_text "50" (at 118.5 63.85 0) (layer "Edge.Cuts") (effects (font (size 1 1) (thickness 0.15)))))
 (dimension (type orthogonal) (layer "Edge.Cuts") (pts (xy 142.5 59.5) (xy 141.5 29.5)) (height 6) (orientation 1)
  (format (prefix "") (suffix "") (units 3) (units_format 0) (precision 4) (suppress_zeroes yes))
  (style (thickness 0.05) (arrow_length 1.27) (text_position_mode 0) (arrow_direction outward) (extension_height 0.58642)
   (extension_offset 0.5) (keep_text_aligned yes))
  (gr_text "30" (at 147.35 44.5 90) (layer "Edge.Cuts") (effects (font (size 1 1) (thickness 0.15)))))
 (segment (start 135.75 43) (end 135.75 45.5) (width 0.2) (layer "F.Cu") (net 1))
 (segment (start 125.75 33) (end 126 33.25) (width 0.2) (layer "F.Cu") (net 1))
 (segment (start 120 52) (end 119.5 51.5) (width 0.2) (layer "F.Cu") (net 1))
 (segment (start 136.2672 50.2328) (end 136.25 50.25) (width 0.2) (layer "F.Cu") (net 1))
 (segment (start 135.6 45.85) (end 135.5 45.75) (width 0.2) (layer "F.Cu") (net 1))
 (segment (start 99.25 43.25) (end 99.5 43.25) (width 0.2) (layer "F.Cu") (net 1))
 (segment (start 135.75 45.5) (end 135.5 45.75) (width 0.2) (layer "F.Cu") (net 1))
 (segment (start 125.75 32) (end 127.82 32) (width 0.2) (layer "F.Cu") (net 1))
 (segment (start 125.75 32) (end 125.75 33) (width 0.2) (layer "F.Cu") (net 1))
 (segment (start 120 52.449999) (end 120 52) (width 0.2) (layer "F.Cu") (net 1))
 (segment (start 127.5 37.915) (end 124.165 37.915) (width 0.2) (layer "F.Cu") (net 1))
 (segment (start 125.5 46) (end 125.75 46.25) (width 0.2) (layer "F.Cu") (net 1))
 (segment (start 120 54) (end 120 52.449999) (width 0.2) (layer "F.Cu") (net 1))
 (segment (start 135.6 47.25) (end 135.6 45.85) (width 0.2) (layer "F.Cu") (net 1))
 (segment (start 137.1425 50.2328) (end 136.2672 50.2328) (width 0.2) (layer "F.Cu") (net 1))
 (segment (start 123.08 32) (end 125.75 32) (width 0.2) (layer "F.Cu") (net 1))
 (segment (start 125.5 43.5) (end 124.5 44.5) (width 0.2) (layer "F.Cu") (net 1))
 (segment (start 124.165 37.915) (end 124 37.75) (width 0.2) (layer "F.Cu") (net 1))
 (segment (start 125.5 45.4375) (end 125.5 46) (width 0.2) (layer "F.Cu") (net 1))
 (segment (start 124.5 44.5) (end 124.25 44.5) (width 0.2) (layer "F.Cu") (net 1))
 (segment (start 98 44.5) (end 99.25 43.25) (width 0.2) (layer "F.Cu") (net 1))
 (via (at 136.25 50.25) (size 0.6) (drill 0.3) (layers "F.Cu" "B.Cu") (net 1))
 (via (at 119.5 51.5) (size 0.6) (drill 0.3) (layers "F.Cu" "B.Cu") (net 1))
 (via (at 124.25 44.5) (size 0.6) (drill 0.3) (layers "F.Cu" "B.Cu") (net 1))
 (via (at 135.5 45.75) (size 0.6) (drill 0.3) (layers "F.Cu" "B.Cu") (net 1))
 (via (at 99.5 43.25) (size 0.6) (drill 0.3) (layers "F.Cu" "B.Cu") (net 1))
 (via (at 125.75 46.25) (size 0.6) (drill 0.3) (layers "F.Cu" "B.Cu") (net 1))
 (via (at 124 37.75) (size 0.6) (drill 0.3) (layers "F.Cu" "B.Cu") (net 1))
 (via (at 126 33.25) (size 0.6) (drill 0.3) (layers "F.Cu" "B.Cu") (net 1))
 (segment (start 137.1425 48.75) (end 135.6 48.75) (width 0.2) (layer "F.Cu") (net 4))
 (segment (start 123.5 39) (end 125.062501 39) (width 0.2) (layer "F.Cu") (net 2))
 (segment (start 118 44.5) (end 123.5 39) (width 0.2) (layer "F.Cu") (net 2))
 (segment (start 127.652501 41.59) (end 127.8 41.59) (width 0.2) (layer "F.Cu") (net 2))
 (segment (start 125.062501 39) (end 127.652501 41.59) (width 0.2) (layer "F.Cu") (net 2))
 (segment (start 129.83 39.015) (end 130.015 39.2) (width 0.2) (layer "F.Cu") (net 5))
 (segment (start 127.5 39.015) (end 129.83 39.015) (width 0.2) (layer "F.Cu") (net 5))
 (segment (start 125.767 44.75) (end 125.0875 44.75) (width 0.2) (layer "F.Cu") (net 8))
 (segment (start 124.4 45.4375) (end 124.4 47.65) (width 0.2) (layer "F.Cu") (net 8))
 (segment (start 126.4 43.1) (end 126.4 44.117) (width 0.2) (layer "F.Cu") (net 8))
 (segment (start 127.09 43.1) (end 126.4 43.1) (width 0.2) (layer "F.Cu") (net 8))
 (segment (start 125.0875 44.75) (end 124.4 45.4375) (width 0.2) (layer "F.Cu") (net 8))
 (segment (start 126.4 44.117) (end 125.767 44.75) (width 0.2) (layer "F.Cu") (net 8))
 (segment (start 124.4 47.65) (end 124.75 48) (width 0.2) (layer "F.Cu") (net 8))
 (segment (start 124.4 43.5) (end 122.250002 45.649998) (width 0.2) (layer "F.Cu") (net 7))
 (segment (start 122.250002 45.649998) (end 122.250002 48) (width 0.2) (layer "F.Cu") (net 7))
 (segment (start 125.2 42.7) (end 124.4 43.5) (width 0.2) (layer "F.Cu") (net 7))
 (segment (start 124.4 43.5) (end 124.4 43.75) (width 0.2) (layer "F.Cu") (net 7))
 (segment (start 127.09 42.7) (end 125.2 42.7) (width 0.2) (layer "F.Cu") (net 7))
 (segment (start 126.54 41.75) (end 127.09 42.3) (width 0.2) (layer "F.Cu") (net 18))
 (segment (start 124.75 41.75) (end 126.54 41.75) (width 0.2) (layer "F.Cu") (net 18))
 (segment (start 126.961 39.711) (end 126.25 39) (width 0.2) (layer "F.Cu") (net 3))
 (segment (start 128.6 41.1) (end 127.211 39.711) (width 0.2) (layer "F.Cu") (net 3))
 (segment (start 128.6 41.59) (end 128.6 41.1) (width 0.2) (layer "F.Cu") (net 3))
 (segment (start 127.211 39.711) (end 126.961 39.711) (width 0.2) (layer "F.Cu") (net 3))
 (segment (start 132.91 43.5) (end 133.5 43.5) (width 0.2) (layer "F.Cu") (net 12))
 (segment (start 133.5 43.5) (end 134 43) (width 0.2) (layer "F.Cu") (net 12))
 (segment (start 134 43) (end 134.65 43) (width 0.2) (layer "F.Cu") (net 12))
 (segment (start 132.91 43.9) (end 134.55 43.9) (width 0.2) (layer "F.Cu") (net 39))
 (segment (start 134.55 43.9) (end 134.65 44) (width 0.2) (layer "F.Cu") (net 39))
 (segment (start 133.755 44.7) (end 132.91 44.7) (width 0.2) (layer "F.Cu") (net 13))
 (segment (start 134.5 48.75) (end 134.5 47.25) (width 0.2) (layer "F.Cu") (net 13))
 (segment (start 134.5 45.445) (end 133.755 44.7) (width 0.2) (layer "F.Cu") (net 13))
 (segment (start 134.5 47.25) (end 134.5 45.445) (width 0.2) (layer "F.Cu") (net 13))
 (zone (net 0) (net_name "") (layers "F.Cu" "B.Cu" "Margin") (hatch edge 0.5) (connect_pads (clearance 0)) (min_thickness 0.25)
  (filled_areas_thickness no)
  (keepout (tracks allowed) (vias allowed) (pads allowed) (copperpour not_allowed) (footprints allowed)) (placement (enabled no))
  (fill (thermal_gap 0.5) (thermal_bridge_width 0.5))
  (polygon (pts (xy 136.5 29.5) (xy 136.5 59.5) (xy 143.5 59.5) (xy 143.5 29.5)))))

